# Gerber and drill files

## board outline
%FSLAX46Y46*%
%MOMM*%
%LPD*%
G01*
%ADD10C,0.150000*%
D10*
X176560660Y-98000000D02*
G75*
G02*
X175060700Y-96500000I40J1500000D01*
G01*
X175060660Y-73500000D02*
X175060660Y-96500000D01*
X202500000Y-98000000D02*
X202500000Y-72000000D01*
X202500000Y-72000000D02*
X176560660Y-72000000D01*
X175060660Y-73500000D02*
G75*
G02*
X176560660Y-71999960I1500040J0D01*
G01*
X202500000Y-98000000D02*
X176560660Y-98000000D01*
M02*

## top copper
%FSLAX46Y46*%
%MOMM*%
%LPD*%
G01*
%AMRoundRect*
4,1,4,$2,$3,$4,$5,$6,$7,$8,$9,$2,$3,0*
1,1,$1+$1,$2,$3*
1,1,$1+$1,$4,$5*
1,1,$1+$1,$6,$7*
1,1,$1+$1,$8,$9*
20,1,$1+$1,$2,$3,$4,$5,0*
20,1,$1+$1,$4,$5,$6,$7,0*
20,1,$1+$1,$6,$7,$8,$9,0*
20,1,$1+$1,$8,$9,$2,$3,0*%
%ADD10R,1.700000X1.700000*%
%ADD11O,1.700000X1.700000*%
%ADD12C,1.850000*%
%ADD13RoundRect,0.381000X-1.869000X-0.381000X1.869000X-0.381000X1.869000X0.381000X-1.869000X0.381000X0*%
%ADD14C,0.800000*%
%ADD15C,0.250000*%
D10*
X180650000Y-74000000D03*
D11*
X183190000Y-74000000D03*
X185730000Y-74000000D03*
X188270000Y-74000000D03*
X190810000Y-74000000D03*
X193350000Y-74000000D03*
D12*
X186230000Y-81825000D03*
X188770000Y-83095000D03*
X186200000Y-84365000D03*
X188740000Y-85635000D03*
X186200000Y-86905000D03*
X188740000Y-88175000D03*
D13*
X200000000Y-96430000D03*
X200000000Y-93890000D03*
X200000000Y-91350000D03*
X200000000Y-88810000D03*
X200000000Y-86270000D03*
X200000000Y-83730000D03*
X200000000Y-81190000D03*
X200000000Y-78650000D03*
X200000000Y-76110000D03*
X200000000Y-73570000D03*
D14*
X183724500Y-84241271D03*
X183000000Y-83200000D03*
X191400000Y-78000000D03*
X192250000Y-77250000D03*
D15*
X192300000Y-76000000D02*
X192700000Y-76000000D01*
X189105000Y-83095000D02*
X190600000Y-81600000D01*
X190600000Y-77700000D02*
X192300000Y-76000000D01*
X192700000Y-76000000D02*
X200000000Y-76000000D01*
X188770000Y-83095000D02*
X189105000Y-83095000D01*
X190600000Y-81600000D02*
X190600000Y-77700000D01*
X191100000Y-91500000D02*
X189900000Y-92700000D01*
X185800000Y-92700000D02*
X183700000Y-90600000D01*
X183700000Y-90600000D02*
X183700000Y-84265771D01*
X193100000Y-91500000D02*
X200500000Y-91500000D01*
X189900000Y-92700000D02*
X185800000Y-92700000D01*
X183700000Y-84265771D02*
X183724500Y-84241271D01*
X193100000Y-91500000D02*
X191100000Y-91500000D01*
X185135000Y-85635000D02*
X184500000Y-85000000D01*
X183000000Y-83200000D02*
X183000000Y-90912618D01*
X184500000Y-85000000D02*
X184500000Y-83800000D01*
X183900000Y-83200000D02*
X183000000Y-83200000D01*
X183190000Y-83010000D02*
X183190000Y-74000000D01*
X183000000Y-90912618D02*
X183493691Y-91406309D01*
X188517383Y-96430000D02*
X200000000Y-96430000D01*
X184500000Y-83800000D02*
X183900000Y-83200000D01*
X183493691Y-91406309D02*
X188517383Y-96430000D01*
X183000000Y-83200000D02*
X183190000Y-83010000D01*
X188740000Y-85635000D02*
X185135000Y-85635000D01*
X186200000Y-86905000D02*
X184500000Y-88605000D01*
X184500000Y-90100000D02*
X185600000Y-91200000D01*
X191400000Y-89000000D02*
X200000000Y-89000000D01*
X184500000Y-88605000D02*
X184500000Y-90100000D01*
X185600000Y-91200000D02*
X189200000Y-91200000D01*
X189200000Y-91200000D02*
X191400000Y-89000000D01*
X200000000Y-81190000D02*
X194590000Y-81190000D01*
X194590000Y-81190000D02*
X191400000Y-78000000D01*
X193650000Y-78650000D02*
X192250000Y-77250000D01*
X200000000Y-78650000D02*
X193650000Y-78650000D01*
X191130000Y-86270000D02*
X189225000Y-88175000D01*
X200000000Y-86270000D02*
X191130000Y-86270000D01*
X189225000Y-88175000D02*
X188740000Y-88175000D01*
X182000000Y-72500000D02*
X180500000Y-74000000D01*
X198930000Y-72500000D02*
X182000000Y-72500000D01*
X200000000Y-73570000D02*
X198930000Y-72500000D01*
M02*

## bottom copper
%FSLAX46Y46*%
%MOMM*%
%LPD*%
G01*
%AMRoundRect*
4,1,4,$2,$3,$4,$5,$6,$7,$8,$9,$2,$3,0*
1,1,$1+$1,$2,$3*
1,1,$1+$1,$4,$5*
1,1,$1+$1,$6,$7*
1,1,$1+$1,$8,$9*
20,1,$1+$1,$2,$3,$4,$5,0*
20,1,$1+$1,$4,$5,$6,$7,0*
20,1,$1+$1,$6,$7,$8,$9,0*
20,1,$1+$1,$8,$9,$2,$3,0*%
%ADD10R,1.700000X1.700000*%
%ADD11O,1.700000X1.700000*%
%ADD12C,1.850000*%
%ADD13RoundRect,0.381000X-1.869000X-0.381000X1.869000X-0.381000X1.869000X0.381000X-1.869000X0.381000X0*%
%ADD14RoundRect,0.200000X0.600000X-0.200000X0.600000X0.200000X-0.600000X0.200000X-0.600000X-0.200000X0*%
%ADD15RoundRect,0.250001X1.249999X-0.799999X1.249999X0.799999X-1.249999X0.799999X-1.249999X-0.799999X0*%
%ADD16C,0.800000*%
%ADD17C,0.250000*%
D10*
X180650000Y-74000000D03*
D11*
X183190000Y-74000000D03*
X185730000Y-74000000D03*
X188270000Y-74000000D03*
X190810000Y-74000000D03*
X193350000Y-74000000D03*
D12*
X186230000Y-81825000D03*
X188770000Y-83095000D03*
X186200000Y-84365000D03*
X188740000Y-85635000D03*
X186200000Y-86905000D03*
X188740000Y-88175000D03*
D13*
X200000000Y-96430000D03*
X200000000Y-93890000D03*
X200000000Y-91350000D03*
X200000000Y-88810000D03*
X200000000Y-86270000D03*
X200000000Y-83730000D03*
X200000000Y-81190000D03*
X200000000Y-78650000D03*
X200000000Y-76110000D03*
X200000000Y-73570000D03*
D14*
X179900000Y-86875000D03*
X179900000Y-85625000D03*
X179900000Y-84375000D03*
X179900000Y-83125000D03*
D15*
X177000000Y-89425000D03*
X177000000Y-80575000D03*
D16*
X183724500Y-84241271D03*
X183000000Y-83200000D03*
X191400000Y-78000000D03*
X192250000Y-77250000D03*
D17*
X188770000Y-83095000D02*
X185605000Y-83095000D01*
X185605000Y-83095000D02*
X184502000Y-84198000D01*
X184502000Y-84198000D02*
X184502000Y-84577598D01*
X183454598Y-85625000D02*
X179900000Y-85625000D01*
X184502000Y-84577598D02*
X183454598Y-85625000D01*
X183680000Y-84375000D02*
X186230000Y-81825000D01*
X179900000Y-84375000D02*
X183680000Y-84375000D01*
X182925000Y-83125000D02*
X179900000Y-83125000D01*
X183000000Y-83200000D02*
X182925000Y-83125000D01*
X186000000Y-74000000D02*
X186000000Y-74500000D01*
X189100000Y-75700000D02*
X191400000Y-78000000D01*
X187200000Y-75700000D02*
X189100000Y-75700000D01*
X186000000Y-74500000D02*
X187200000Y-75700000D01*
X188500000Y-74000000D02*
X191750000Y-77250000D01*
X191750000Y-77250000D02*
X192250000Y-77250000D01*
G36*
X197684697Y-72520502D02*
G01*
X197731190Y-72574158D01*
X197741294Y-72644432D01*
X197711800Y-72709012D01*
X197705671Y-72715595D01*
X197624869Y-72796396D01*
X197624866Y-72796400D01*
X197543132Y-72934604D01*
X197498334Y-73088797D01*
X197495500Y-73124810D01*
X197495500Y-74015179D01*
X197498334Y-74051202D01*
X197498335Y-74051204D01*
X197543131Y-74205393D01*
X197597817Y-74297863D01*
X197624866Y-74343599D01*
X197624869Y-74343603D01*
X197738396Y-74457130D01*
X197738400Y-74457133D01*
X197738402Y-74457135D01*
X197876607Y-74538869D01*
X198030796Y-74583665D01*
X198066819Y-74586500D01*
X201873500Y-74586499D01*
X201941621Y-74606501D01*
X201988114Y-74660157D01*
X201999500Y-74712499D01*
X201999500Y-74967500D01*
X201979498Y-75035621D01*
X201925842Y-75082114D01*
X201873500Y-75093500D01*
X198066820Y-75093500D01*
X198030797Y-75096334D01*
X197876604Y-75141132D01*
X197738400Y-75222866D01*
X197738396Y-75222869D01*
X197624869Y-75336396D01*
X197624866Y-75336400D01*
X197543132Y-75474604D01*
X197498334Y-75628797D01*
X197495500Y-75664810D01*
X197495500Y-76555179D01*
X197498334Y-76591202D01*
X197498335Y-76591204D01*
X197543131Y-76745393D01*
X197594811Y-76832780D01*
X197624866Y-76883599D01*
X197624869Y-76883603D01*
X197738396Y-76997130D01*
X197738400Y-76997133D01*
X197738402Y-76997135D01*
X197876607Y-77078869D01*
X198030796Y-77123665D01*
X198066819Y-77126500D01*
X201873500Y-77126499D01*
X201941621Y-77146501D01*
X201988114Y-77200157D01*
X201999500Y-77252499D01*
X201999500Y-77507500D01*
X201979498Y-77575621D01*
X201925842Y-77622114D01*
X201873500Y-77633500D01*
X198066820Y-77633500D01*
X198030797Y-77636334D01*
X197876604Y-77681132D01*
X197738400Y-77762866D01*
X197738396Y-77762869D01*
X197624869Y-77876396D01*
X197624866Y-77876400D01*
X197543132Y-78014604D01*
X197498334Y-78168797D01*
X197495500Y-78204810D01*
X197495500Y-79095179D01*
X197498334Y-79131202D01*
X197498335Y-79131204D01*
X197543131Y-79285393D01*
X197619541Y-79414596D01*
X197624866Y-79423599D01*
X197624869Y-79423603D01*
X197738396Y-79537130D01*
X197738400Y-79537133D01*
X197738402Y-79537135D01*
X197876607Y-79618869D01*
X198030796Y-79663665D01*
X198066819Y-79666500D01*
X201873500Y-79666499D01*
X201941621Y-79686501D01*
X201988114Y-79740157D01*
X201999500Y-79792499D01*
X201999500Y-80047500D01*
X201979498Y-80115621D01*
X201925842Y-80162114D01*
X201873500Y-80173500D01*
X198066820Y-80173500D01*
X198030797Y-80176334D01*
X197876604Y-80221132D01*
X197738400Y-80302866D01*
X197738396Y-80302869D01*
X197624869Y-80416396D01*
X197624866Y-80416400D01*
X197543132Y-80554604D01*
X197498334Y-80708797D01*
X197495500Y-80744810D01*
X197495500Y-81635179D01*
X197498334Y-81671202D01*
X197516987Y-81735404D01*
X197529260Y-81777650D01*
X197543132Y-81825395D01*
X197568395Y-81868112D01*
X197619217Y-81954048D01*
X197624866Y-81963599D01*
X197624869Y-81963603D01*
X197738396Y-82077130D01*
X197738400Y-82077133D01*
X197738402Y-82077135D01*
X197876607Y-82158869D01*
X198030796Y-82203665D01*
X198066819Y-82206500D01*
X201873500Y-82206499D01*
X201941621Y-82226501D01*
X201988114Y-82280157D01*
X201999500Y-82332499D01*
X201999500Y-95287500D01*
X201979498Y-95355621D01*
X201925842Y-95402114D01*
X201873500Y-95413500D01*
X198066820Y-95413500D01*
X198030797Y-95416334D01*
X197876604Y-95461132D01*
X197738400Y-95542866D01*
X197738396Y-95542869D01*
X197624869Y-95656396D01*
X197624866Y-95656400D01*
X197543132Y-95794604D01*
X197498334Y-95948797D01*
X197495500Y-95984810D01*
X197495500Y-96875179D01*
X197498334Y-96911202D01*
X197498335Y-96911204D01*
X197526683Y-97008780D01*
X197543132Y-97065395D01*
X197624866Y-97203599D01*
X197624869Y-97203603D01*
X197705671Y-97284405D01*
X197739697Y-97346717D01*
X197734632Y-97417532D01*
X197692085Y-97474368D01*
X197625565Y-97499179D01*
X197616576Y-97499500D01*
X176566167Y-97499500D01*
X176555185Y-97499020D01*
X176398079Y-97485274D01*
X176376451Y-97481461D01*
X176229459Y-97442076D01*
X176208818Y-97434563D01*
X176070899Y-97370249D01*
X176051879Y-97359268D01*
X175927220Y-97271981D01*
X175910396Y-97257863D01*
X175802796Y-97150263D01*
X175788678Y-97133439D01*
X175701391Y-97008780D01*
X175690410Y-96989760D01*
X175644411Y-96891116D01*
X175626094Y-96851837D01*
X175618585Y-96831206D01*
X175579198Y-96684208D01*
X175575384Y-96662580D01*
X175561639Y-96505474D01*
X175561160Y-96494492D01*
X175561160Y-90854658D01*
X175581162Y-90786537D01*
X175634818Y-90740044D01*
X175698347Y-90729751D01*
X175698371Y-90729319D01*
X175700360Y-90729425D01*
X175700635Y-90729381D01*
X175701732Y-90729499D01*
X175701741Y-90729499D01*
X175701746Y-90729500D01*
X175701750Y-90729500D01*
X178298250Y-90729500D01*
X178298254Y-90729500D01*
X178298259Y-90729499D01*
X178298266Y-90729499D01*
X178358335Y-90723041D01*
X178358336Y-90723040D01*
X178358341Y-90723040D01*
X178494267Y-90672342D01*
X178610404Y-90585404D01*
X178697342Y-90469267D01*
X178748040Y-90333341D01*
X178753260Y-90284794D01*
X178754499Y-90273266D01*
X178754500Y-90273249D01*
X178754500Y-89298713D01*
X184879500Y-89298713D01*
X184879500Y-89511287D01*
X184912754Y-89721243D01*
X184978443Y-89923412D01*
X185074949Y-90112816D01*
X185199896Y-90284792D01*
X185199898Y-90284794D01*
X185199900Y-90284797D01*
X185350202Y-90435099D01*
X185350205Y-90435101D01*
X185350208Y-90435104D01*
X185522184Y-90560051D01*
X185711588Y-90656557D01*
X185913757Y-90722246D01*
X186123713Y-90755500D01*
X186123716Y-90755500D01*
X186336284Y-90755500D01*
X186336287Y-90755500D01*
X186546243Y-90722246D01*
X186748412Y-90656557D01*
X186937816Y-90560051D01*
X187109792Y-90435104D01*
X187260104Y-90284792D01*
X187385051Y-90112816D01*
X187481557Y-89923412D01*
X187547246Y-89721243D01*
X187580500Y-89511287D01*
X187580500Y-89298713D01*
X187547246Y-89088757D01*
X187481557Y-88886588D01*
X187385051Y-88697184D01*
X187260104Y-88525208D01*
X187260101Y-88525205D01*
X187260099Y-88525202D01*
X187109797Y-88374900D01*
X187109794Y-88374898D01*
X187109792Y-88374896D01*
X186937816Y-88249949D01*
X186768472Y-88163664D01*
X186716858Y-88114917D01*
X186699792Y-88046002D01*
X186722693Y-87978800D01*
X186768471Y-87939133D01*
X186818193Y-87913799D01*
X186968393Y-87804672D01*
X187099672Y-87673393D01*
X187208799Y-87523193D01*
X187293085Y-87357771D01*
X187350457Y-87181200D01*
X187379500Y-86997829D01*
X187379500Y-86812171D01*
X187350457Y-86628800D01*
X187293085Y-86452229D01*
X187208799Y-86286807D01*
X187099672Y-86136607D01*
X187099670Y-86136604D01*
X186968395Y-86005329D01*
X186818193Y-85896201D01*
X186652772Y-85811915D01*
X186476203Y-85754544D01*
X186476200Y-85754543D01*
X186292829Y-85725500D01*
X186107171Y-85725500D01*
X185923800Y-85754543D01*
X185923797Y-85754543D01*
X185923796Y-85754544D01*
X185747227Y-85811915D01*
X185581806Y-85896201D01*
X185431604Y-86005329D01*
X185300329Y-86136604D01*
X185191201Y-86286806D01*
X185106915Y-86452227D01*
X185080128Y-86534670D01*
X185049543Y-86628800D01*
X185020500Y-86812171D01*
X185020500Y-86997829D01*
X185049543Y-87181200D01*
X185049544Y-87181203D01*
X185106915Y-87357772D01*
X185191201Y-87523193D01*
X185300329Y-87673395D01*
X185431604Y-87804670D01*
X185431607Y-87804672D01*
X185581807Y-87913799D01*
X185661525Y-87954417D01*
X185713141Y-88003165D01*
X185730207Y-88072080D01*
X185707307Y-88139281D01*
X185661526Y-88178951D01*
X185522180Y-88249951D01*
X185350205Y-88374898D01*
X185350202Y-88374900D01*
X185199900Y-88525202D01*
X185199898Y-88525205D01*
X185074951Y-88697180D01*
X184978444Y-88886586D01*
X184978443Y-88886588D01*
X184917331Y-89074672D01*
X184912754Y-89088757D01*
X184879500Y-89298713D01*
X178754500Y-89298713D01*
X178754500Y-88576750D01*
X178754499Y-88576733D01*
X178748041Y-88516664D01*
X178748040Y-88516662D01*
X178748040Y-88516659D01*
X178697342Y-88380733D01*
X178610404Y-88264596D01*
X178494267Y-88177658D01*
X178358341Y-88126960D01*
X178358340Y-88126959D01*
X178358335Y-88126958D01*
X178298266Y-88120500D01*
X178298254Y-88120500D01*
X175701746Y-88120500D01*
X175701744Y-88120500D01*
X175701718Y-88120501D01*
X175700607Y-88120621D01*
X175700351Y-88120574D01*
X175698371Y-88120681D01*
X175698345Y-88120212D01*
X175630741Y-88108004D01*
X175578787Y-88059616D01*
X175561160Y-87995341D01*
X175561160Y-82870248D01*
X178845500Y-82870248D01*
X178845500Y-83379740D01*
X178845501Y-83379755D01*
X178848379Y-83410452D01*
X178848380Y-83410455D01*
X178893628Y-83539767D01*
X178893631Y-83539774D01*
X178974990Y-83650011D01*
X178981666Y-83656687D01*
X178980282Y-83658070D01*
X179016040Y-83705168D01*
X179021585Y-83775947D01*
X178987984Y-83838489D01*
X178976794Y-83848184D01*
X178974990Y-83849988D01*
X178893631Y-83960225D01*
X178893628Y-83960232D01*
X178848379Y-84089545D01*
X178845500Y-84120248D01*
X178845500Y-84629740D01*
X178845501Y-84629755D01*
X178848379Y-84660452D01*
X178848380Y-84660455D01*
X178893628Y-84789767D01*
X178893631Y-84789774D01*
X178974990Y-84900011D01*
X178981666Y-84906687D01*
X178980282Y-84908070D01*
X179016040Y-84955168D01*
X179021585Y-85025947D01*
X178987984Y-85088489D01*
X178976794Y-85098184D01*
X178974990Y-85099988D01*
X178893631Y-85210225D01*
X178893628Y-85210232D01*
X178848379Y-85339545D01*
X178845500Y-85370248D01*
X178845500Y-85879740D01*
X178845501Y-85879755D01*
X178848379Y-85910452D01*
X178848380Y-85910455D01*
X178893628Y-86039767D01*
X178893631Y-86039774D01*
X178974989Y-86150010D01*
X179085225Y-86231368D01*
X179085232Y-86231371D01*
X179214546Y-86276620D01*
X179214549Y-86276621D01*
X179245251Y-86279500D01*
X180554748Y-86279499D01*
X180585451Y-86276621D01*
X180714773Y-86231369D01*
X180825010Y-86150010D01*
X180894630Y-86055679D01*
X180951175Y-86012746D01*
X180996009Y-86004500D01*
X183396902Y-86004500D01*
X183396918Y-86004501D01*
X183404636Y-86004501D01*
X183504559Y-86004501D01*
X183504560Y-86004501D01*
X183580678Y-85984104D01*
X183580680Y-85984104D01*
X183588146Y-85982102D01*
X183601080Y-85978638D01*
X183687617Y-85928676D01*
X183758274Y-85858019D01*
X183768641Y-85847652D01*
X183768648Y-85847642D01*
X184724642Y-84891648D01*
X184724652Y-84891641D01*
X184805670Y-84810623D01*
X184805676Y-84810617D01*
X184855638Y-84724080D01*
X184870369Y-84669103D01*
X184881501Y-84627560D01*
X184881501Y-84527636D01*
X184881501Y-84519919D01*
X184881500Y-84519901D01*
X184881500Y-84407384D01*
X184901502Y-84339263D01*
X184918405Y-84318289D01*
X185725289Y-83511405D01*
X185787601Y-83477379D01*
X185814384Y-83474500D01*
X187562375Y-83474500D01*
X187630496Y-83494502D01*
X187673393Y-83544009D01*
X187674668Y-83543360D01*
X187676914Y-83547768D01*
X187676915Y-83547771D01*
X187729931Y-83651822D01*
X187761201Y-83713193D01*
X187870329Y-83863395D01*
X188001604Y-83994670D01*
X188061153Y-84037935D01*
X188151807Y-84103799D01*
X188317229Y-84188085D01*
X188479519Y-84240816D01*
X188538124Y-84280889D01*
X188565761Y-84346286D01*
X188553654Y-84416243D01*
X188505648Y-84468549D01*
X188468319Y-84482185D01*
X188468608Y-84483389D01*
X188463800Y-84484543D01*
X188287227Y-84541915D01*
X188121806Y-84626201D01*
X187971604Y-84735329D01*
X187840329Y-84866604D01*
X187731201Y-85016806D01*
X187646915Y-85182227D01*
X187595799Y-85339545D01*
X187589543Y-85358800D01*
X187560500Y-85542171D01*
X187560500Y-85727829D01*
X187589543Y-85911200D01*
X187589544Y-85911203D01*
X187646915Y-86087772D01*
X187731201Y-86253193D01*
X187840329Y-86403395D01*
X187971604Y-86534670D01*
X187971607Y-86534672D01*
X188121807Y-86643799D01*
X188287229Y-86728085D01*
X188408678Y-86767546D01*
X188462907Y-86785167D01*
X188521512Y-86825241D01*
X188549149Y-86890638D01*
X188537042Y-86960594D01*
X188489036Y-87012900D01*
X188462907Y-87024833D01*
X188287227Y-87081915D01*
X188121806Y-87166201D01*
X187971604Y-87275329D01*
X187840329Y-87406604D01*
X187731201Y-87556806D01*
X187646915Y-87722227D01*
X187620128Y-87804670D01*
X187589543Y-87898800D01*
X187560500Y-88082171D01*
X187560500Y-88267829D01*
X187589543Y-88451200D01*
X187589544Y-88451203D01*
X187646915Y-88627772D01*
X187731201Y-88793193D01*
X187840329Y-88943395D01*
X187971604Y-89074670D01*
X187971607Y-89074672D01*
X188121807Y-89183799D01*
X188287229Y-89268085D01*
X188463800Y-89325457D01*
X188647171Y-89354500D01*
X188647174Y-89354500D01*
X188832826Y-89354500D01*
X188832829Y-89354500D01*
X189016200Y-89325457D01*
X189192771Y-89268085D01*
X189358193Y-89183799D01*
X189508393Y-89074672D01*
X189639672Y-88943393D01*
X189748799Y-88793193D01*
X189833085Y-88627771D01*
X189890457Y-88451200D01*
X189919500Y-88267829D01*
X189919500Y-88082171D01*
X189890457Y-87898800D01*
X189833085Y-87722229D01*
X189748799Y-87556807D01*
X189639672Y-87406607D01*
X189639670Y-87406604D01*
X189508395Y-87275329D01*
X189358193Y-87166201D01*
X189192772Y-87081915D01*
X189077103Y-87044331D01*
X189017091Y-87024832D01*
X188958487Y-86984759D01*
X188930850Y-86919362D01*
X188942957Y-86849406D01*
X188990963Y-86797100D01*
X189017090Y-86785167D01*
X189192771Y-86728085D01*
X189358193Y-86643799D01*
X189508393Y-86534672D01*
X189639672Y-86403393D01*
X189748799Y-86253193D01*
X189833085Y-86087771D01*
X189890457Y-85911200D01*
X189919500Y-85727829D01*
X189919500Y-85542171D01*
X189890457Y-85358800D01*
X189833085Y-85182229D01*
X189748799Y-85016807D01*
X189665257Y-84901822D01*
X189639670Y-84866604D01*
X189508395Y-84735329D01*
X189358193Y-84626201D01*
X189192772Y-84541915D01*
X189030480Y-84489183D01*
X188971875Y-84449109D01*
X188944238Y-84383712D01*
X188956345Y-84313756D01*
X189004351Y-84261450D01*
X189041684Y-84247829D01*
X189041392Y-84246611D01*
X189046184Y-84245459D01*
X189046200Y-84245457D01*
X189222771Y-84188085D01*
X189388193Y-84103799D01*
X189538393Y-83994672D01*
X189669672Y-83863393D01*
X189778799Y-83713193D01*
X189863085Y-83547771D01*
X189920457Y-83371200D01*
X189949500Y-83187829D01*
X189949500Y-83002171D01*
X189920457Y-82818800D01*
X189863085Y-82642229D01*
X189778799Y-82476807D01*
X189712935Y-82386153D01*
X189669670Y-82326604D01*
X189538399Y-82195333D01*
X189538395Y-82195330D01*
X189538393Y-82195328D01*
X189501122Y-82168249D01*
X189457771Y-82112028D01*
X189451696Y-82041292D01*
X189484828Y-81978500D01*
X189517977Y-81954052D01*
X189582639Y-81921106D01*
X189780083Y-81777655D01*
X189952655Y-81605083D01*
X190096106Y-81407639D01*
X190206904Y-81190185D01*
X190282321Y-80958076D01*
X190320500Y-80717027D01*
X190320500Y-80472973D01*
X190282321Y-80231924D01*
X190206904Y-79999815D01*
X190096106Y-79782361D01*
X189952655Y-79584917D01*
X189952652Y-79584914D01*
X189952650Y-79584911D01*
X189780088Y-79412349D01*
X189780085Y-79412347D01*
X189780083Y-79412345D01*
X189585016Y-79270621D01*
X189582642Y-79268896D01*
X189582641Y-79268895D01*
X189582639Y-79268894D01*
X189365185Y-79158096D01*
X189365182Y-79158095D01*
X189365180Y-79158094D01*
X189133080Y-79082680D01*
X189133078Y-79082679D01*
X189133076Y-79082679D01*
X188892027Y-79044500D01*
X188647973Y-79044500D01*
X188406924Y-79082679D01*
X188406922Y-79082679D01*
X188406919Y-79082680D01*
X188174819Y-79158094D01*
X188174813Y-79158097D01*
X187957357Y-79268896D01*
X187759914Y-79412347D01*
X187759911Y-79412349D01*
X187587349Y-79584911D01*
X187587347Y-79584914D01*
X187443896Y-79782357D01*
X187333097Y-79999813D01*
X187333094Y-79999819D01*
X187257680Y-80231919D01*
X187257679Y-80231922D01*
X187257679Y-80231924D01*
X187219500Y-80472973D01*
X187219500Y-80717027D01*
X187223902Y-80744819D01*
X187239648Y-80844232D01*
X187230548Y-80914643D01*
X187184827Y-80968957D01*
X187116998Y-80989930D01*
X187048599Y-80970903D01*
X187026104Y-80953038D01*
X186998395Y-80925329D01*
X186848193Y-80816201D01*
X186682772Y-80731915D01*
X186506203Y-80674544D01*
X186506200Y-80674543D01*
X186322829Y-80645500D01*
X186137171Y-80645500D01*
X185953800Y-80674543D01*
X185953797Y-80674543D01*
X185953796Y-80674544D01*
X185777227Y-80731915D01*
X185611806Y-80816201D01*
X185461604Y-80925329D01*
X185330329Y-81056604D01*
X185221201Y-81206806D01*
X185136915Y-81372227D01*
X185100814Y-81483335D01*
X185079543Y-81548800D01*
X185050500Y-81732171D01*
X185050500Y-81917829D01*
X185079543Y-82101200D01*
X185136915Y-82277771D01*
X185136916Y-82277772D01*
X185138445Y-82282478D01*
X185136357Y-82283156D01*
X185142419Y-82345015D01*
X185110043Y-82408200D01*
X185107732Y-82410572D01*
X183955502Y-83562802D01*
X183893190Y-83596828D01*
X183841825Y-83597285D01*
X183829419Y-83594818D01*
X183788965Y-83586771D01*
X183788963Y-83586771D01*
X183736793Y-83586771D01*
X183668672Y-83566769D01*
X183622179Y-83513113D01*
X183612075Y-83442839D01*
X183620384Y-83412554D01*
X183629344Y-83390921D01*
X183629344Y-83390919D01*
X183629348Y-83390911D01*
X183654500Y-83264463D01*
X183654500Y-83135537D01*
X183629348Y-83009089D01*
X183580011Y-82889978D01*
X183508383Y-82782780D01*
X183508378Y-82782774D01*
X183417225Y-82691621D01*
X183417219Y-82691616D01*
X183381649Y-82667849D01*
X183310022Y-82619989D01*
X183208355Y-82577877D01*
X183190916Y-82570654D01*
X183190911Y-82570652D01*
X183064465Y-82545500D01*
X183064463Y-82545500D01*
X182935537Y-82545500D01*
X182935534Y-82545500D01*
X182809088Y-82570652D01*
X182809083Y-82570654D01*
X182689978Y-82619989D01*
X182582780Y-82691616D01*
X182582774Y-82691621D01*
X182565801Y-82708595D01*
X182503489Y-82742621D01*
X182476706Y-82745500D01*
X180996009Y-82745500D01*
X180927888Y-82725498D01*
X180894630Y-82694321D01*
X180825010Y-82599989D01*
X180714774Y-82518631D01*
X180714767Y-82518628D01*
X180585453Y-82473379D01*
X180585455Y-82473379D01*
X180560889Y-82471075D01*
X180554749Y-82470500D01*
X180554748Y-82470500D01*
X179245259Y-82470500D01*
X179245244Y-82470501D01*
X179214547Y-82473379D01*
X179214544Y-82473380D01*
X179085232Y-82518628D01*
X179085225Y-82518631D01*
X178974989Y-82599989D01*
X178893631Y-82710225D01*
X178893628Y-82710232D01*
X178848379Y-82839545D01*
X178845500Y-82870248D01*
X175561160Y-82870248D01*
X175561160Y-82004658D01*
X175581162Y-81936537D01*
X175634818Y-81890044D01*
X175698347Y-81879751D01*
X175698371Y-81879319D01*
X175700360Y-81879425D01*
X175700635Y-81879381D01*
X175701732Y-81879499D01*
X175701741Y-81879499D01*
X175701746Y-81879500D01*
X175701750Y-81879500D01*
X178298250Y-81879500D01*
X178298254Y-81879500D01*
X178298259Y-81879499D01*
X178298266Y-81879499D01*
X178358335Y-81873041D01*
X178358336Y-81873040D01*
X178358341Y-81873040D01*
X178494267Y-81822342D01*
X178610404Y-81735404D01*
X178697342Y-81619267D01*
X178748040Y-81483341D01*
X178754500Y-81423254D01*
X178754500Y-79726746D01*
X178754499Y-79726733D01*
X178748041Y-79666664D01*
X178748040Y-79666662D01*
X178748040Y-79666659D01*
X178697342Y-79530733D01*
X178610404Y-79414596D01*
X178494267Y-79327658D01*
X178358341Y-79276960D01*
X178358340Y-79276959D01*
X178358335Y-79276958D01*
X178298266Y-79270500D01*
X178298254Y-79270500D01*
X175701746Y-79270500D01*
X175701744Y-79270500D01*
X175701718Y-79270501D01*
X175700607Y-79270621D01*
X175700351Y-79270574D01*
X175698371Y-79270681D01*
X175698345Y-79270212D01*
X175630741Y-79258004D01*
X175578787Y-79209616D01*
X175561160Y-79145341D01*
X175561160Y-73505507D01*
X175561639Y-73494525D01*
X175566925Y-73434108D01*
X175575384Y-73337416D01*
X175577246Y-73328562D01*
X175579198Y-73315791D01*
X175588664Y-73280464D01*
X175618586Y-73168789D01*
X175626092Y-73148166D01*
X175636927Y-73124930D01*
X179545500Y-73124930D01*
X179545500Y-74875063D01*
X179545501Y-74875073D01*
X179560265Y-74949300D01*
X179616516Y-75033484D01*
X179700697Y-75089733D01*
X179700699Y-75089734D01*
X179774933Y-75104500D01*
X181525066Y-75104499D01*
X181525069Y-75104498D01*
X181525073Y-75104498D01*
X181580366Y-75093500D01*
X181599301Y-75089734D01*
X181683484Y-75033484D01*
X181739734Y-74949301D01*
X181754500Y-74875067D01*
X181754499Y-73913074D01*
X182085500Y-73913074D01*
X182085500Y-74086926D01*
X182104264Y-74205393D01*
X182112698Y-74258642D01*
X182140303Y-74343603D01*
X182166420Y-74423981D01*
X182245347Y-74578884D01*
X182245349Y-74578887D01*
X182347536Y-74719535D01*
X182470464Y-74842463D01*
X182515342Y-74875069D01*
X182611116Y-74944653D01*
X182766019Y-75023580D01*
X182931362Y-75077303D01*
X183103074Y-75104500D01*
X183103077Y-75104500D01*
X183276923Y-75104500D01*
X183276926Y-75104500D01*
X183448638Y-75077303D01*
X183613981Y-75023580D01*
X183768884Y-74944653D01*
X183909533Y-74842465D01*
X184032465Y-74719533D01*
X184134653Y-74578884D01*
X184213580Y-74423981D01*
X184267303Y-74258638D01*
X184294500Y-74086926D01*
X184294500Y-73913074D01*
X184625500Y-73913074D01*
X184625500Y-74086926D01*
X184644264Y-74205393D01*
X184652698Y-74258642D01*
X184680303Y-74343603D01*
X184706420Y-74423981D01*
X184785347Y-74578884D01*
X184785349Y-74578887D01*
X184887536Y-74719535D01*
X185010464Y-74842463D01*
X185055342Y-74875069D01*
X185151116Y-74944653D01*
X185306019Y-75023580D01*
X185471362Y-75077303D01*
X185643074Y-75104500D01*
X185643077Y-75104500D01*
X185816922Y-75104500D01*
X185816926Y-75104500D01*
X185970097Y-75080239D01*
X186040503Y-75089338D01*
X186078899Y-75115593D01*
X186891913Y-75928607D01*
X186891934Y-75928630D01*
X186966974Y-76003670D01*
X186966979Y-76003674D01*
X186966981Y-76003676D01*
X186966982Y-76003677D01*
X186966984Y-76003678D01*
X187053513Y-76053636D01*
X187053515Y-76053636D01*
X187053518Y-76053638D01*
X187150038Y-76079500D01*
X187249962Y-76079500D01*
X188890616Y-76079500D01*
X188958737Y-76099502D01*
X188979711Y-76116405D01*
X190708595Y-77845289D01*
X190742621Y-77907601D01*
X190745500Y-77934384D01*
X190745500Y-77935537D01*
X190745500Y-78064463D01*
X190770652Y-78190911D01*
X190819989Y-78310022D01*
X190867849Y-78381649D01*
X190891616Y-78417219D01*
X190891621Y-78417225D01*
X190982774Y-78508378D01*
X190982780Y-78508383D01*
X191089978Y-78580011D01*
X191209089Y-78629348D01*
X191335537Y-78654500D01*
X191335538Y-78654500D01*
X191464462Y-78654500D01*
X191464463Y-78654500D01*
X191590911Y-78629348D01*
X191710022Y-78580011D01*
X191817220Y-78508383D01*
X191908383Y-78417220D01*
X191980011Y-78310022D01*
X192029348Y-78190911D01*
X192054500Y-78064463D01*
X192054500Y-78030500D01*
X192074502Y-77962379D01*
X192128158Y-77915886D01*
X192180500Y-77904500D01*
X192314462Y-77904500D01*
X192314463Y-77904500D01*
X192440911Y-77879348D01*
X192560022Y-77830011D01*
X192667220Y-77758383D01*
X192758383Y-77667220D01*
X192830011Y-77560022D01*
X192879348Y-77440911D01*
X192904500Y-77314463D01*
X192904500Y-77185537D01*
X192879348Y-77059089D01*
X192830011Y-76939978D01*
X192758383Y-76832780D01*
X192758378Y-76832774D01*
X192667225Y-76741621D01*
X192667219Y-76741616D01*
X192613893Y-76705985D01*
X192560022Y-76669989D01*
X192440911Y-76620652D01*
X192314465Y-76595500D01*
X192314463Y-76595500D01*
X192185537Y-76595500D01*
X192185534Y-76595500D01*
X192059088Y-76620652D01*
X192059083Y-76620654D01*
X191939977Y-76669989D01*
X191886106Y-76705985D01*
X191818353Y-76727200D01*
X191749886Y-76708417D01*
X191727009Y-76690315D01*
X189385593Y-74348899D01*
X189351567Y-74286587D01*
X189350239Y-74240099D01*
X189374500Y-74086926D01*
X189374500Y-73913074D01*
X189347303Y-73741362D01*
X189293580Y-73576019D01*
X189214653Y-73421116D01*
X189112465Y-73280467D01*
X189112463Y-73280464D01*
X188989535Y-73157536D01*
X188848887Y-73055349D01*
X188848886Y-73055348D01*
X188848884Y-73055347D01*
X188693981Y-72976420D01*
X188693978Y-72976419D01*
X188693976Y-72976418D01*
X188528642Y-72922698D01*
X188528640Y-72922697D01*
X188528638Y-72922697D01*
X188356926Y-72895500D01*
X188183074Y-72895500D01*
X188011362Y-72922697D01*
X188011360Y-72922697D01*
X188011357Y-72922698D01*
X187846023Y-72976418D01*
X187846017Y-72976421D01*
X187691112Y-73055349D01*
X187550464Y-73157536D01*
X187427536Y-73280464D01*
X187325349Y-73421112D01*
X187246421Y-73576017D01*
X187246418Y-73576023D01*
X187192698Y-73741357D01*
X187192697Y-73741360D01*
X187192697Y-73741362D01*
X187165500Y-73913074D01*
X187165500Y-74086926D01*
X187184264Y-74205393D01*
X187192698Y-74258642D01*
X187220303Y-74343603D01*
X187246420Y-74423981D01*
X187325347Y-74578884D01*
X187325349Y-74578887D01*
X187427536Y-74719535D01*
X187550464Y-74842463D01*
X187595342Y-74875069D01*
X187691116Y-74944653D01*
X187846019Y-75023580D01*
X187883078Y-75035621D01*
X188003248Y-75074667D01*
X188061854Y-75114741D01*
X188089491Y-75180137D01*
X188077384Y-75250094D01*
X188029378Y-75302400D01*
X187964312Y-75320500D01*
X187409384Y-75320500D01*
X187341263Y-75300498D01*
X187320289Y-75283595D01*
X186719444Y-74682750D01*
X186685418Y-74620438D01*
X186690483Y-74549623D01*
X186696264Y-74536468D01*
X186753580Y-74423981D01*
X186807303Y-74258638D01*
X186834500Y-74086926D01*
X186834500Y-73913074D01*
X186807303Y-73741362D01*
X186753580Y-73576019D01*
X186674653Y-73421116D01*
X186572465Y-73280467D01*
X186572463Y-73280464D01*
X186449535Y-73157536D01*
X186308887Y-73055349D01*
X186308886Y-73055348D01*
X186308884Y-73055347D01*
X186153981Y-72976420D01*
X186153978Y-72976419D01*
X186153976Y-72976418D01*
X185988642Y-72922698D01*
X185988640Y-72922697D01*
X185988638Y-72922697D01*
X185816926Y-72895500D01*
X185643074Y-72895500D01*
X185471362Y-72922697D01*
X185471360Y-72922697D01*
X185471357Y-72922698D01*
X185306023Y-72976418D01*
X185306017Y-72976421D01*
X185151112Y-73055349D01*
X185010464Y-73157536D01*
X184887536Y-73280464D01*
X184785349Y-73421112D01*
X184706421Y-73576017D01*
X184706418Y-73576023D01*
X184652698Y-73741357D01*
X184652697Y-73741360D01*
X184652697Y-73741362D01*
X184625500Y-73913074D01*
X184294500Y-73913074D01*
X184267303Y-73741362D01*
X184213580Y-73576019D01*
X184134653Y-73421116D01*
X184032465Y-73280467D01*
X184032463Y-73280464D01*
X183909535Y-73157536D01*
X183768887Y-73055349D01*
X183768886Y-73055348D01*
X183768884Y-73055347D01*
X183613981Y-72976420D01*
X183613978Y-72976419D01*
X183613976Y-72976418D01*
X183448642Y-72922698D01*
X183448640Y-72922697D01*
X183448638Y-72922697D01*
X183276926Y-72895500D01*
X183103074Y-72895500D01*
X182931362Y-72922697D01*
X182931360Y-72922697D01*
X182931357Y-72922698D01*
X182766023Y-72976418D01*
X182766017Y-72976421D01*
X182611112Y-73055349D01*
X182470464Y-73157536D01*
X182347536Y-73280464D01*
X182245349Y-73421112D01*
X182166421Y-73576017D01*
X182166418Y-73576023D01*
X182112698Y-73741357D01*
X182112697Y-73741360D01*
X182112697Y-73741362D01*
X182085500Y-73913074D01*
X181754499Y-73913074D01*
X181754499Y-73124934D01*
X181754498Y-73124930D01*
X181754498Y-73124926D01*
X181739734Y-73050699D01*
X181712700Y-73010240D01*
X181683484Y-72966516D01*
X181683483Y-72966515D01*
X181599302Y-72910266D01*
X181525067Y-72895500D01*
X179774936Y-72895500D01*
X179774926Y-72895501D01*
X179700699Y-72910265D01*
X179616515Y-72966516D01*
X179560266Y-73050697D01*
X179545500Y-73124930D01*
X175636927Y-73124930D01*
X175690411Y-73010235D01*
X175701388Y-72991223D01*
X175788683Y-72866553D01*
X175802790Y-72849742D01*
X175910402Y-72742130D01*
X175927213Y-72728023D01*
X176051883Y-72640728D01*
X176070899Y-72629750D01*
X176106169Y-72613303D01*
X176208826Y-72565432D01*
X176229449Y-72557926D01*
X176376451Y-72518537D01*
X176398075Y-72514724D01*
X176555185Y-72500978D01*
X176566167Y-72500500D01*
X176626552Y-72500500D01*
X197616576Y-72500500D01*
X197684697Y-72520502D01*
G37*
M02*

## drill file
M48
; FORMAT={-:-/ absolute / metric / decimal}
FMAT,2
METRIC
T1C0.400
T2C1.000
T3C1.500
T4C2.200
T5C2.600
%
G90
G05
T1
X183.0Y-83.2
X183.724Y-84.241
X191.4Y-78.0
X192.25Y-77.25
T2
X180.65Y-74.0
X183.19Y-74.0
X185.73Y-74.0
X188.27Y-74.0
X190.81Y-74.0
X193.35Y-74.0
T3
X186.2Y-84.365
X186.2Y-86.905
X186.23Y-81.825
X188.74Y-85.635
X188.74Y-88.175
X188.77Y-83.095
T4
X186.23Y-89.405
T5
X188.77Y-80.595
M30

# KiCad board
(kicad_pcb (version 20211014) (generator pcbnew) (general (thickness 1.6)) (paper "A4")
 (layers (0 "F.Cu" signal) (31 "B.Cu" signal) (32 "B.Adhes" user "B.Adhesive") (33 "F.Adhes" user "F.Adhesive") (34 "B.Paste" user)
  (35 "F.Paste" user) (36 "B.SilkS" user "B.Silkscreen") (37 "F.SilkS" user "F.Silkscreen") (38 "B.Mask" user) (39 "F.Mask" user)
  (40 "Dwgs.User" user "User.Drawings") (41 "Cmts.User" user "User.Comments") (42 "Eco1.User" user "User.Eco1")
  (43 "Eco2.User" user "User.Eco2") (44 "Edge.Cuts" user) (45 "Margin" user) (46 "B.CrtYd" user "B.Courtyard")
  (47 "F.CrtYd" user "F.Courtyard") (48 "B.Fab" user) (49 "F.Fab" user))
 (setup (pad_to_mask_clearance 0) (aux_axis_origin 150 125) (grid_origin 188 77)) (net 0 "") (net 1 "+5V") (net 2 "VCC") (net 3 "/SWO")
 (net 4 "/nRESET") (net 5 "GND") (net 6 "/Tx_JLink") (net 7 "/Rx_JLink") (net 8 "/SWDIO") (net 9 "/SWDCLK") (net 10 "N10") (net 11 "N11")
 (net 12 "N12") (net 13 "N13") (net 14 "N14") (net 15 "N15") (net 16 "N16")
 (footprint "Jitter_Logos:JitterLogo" (layer "F.Cu") (at 179.25 90)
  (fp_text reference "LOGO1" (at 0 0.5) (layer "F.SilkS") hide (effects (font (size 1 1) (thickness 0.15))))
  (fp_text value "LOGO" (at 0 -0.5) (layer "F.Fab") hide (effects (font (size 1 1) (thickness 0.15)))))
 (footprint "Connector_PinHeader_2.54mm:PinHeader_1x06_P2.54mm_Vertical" (layer "F.Cu") (at 180.65 74 90)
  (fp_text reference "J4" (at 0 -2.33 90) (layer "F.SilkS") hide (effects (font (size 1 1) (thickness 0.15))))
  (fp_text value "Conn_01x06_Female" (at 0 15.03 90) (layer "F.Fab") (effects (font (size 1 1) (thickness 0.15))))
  (pad "1" thru_hole rect (at 0 0 90) (size 1.7 1.7) (drill 1) (layers *.Cu *.Mask) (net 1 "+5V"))
  (pad "2" thru_hole oval (at 0 2.54 90) (size 1.7 1.7) (drill 1) (layers *.Cu *.Mask) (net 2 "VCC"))
  (pad "3" thru_hole oval (at 0 5.08 90) (size 1.7 1.7) (drill 1) (layers *.Cu *.Mask) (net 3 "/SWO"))
  (pad "4" thru_hole oval (at 0 7.62 90) (size 1.7 1.7) (drill 1) (layers *.Cu *.Mask) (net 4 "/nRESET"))
  (pad "5" thru_hole oval (at 0 10.16 90) (size 1.7 1.7) (drill 1) (layers *.Cu *.Mask) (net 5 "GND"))
  (pad "6" thru_hole oval (at 0 12.7 90) (size 1.7 1.7) (drill 1) (layers *.Cu *.Mask) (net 5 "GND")))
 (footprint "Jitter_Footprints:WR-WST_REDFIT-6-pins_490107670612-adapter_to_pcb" (layer "F.Cu") (at 187.5 85 90)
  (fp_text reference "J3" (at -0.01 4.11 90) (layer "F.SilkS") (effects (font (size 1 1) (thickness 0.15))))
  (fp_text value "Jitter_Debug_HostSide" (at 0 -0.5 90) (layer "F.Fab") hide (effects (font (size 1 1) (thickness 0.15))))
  (pad "" np_thru_hole circle locked (at 4.405 1.27 90) (size 2.6 2.6) (drill 2.6) (layers *.Cu *.Mask))
  (pad "" np_thru_hole circle locked (at -4.405 -1.27 90) (size 2.2 2.2) (drill 2.2) (layers *.Cu *.Mask))
  (pad "1" thru_hole circle locked (at 3.175 -1.27 90) (size 1.85 1.85) (drill 1.5) (layers *.Cu *.Mask) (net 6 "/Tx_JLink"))
  (pad "2" thru_hole circle locked (at 1.905 1.27 90) (size 1.85 1.85) (drill 1.5) (layers *.Cu *.Mask) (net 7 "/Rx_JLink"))
  (pad "3" thru_hole circle locked (at 0.635 -1.3 90) (size 1.85 1.85) (drill 1.5) (layers *.Cu *.Mask) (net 5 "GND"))
  (pad "4" thru_hole circle locked (at -0.635 1.24 90) (size 1.85 1.85) (drill 1.5) (layers *.Cu *.Mask) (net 2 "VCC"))
  (pad "5" thru_hole circle locked (at -1.905 -1.3 90) (size 1.85 1.85) (drill 1.5) (layers *.Cu *.Mask) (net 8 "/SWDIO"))
  (pad "6" thru_hole circle locked (at -3.175 1.24 90) (size 1.85 1.85) (drill 1.5) (layers *.Cu *.Mask) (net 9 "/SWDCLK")))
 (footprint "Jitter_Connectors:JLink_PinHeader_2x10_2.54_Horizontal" (layer "F.Cu") (at 200 85)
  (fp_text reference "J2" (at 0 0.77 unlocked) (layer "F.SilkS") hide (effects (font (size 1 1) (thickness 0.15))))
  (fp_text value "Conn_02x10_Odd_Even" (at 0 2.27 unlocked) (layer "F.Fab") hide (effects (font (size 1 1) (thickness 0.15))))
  (pad "1" smd roundrect (at 0 11.43) (size 4.5 1.524) (layers "F.Cu" "F.Paste" "F.Mask") (roundrect_rratio 0.25) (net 2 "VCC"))
  (pad "2" smd roundrect (at 0 11.43) (size 4.5 1.524) (layers "B.Cu" "B.Paste" "B.Mask") (roundrect_rratio 0.25) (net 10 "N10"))
  (pad "3" smd roundrect (at 0 8.89) (size 4.5 1.524) (layers "F.Cu" "F.Paste" "F.Mask") (roundrect_rratio 0.25) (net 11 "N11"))
  (pad "4" smd roundrect (at 0 8.89) (size 4.5 1.524) (layers "B.Cu" "B.Paste" "B.Mask") (roundrect_rratio 0.25) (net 5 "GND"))
  (pad "5" smd roundrect (at 0 6.35) (size 4.5 1.524) (layers "F.Cu" "F.Paste" "F.Mask") (roundrect_rratio 0.25) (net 6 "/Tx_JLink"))
  (pad "6" smd roundrect (at 0 6.35) (size 4.5 1.524) (layers "B.Cu" "B.Paste" "B.Mask") (roundrect_rratio 0.25) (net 5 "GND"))
  (pad "7" smd roundrect (at 0 3.81) (size 4.5 1.524) (layers "F.Cu" "F.Paste" "F.Mask") (roundrect_rratio 0.25) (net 8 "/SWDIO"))
  (pad "8" smd roundrect (at 0 3.81) (size 4.5 1.524) (layers "B.Cu" "B.Paste" "B.Mask") (roundrect_rratio 0.25) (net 5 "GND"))
  (pad "9" smd roundrect (at 0 1.27) (size 4.5 1.524) (layers "F.Cu" "F.Paste" "F.Mask") (roundrect_rratio 0.25) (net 9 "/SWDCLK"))
  (pad "10" smd roundrect (at 0 1.27) (size 4.5 1.524) (layers "B.Cu" "B.Paste" "B.Mask") (roundrect_rratio 0.25) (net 5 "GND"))
  (pad "11" smd roundrect (at 0 -1.27) (size 4.5 1.524) (layers "F.Cu" "F.Paste" "F.Mask") (roundrect_rratio 0.25) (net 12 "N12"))
  (pad "12" smd roundrect (at 0 -1.27) (size 4.5 1.524) (layers "B.Cu" "B.Paste" "B.Mask") (roundrect_rratio 0.25) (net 5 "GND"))
  (pad "13" smd roundrect (at 0 -3.81) (size 4.5 1.524) (layers "F.Cu" "F.Paste" "F.Mask") (roundrect_rratio 0.25) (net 3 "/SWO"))
  (pad "14" smd roundrect (at 0 -3.81) (size 4.5 1.524) (layers "B.Cu" "B.Paste" "B.Mask") (roundrect_rratio 0.25) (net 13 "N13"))
  (pad "15" smd roundrect (at 0 -6.35) (size 4.5 1.524) (layers "F.Cu" "F.Paste" "F.Mask") (roundrect_rratio 0.25) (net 4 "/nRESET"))
  (pad "16" smd roundrect (at 0 -6.35) (size 4.5 1.524) (layers "B.Cu" "B.Paste" "B.Mask") (roundrect_rratio 0.25) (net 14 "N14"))
  (pad "17" smd roundrect (at 0 -8.89) (size 4.5 1.524) (layers "F.Cu" "F.Paste" "F.Mask") (roundrect_rratio 0.25) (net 7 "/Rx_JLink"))
  (pad "18" smd roundrect (at 0 -8.89) (size 4.5 1.524) (layers "B.Cu" "B.Paste" "B.Mask") (roundrect_rratio 0.25) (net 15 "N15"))
  (pad "19" smd roundrect (at 0 -11.43) (size 4.5 1.524) (layers "F.Cu" "F.Paste" "F.Mask") (roundrect_rratio 0.25) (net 1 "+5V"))
  (pad "20" smd roundrect (at 0 -11.43) (size 4.5 1.524) (layers "B.Cu" "B.Paste" "B.Mask") (roundrect_rratio 0.25) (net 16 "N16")))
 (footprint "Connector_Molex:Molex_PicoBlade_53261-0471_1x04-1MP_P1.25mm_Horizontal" (layer "B.Cu") (at 177.5 85 90)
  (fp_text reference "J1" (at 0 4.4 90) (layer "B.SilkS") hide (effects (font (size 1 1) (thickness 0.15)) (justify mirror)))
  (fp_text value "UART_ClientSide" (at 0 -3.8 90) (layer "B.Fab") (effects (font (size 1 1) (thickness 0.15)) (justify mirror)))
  (pad "1" smd roundrect (at -1.875 2.4 90) (size 0.8 1.6) (layers "B.Cu" "B.Paste" "B.Mask") (roundrect_rratio 0.25) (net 5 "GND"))
  (pad "2" smd roundrect (at -0.625 2.4 90) (size 0.8 1.6) (layers "B.Cu" "B.Paste" "B.Mask") (roundrect_rratio 0.25) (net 7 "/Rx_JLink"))
  (pad "3" smd roundrect (at 0.625 2.4 90) (size 0.8 1.6) (layers "B.Cu" "B.Paste" "B.Mask") (roundrect_rratio 0.25) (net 6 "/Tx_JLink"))
  (pad "4" smd roundrect (at 1.875 2.4 90) (size 0.8 1.6) (layers "B.Cu" "B.Paste" "B.Mask") (roundrect_rratio 0.25) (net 2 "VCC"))
  (pad "MP" smd roundrect (at -4.425 -0.5 90) (size 2.1 3) (layers "B.Cu" "B.Paste" "B.Mask") (roundrect_rratio 0.1190480952))
  (pad "MP" smd roundrect (at 4.425 -0.5 90) (size 2.1 3) (layers "B.Cu" "B.Paste" "B.Mask") (roundrect_rratio 0.1190480952)))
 (gr_arc (start 176.56066 98) (mid 175.5 97.56066) (end 175.06066 96.5) (layer "Edge.Cuts") (width 0.15))
 (gr_line (start 175.06066 73.5) (end 175.06066 96.5) (layer "Edge.Cuts") (width 0.15))
 (gr_line (start 202.5 98) (end 202.5 72) (layer "Edge.Cuts") (width 0.15))
 (gr_line (start 202.5 72) (end 176.56066 72) (layer "Edge.Cuts") (width 0.15))
 (gr_arc (start 175.06066 73.5) (mid 175.5 72.43934) (end 176.56066 72) (layer "Edge.Cuts") (width 0.15))
 (gr_line (start 202.5 98) (end 176.56066 98) (layer "Edge.Cuts") (width 0.15))
 (segment (start 192.3 76) (end 192.7 76) (width 0.25) (layer "F.Cu") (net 7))
 (segment (start 189.105 83.095) (end 190.6 81.6) (width 0.25) (layer "F.Cu") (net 7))
 (segment (start 190.6 77.7) (end 192.3 76) (width 0.25) (layer "F.Cu") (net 7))
 (segment (start 192.7 76) (end 200 76) (width 0.25) (layer "F.Cu") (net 7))
 (segment (start 188.77 83.095) (end 189.105 83.095) (width 0.25) (layer "F.Cu") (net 7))
 (segment (start 190.6 81.6) (end 190.6 77.7) (width 0.25) (layer "F.Cu") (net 7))
 (segment (start 188.77 83.095) (end 185.605 83.095) (width 0.25) (layer "B.Cu") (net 7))
 (segment (start 185.605 83.095) (end 184.502 84.198) (width 0.25) (layer "B.Cu") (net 7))
 (segment (start 184.502 84.198) (end 184.502 84.577598) (width 0.25) (layer "B.Cu") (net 7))
 (segment (start 183.454598 85.625) (end 179.9 85.625) (width 0.25) (layer "B.Cu") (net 7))
 (segment (start 184.502 84.577598) (end 183.454598 85.625) (width 0.25) (layer "B.Cu") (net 7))
 (segment (start 191.1 91.5) (end 189.9 92.7) (width 0.25) (layer "F.Cu") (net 6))
 (segment (start 185.8 92.7) (end 183.7 90.6) (width 0.25) (layer "F.Cu") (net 6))
 (segment (start 183.7 90.6) (end 183.7 84.265771) (width 0.25) (layer "F.Cu") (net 6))
 (segment (start 193.1 91.5) (end 200.5 91.5) (width 0.25) (layer "F.Cu") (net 6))
 (segment (start 189.9 92.7) (end 185.8 92.7) (width 0.25) (layer "F.Cu") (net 6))
 (segment (start 183.7 84.265771) (end 183.7245 84.241271) (width 0.25) (layer "F.Cu") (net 6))
 (segment (start 193.1 91.5) (end 191.1 91.5) (width 0.25) (layer "F.Cu") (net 6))
 (via (at 183.7245 84.241271) (size 0.8) (drill 0.4) (layers "F.Cu" "B.Cu") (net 6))
 (segment (start 183.68 84.375) (end 186.23 81.825) (width 0.25) (layer "B.Cu") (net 6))
 (segment (start 179.9 84.375) (end 183.68 84.375) (width 0.25) (layer "B.Cu") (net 6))
 (segment (start 185.135 85.635) (end 184.5 85) (width 0.25) (layer "F.Cu") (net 2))
 (segment (start 183 83.2) (end 183 90.912618) (width 0.25) (layer "F.Cu") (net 2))
 (segment (start 184.5 85) (end 184.5 83.8) (width 0.25) (layer "F.Cu") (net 2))
 (segment (start 183.9 83.2) (end 183 83.2) (width 0.25) (layer "F.Cu") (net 2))
 (segment (start 183.19 83.01) (end 183.19 74) (width 0.25) (layer "F.Cu") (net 2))
 (segment (start 183 90.912618) (end 183.493691 91.406309) (width 0.25) (layer "F.Cu") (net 2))
 (segment (start 188.517383 96.43) (end 200 96.43) (width 0.25) (layer "F.Cu") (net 2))
 (segment (start 184.5 83.8) (end 183.9 83.2) (width 0.25) (layer "F.Cu") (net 2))
 (segment (start 183.493691 91.406309) (end 188.517383 96.43) (width 0.25) (layer "F.Cu") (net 2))
 (segment (start 183 83.2) (end 183.19 83.01) (width 0.25) (layer "F.Cu") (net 2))
 (segment (start 188.74 85.635) (end 185.135 85.635) (width 0.25) (layer "F.Cu") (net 2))
 (via (at 183 83.2) (size 0.8) (drill 0.4) (layers "F.Cu" "B.Cu") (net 2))
 (segment (start 182.925 83.125) (end 179.9 83.125) (width 0.25) (layer "B.Cu") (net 2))
 (segment (start 183 83.2) (end 182.925 83.125) (width 0.25) (layer "B.Cu") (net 2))
 (segment (start 186.2 86.905) (end 184.5 88.605) (width 0.25) (layer "F.Cu") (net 8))
 (segment (start 184.5 90.1) (end 185.6 91.2) (width 0.25) (layer "F.Cu") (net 8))
 (segment (start 191.4 89) (end 200 89) (width 0.25) (layer "F.Cu") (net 8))
 (segment (start 184.5 88.605) (end 184.5 90.1) (width 0.25) (layer "F.Cu") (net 8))
 (segment (start 185.6 91.2) (end 189.2 91.2) (width 0.25) (layer "F.Cu") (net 8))
 (segment (start 189.2 91.2) (end 191.4 89) (width 0.25) (layer "F.Cu") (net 8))
 (segment (start 200 81.19) (end 194.59 81.19) (width 0.25) (layer "F.Cu") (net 3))
 (segment (start 194.59 81.19) (end 191.4 78) (width 0.25) (layer "F.Cu") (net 3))
 (via (at 191.4 78) (size 0.8) (drill 0.4) (layers "F.Cu" "B.Cu") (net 3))
 (segment (start 186 74) (end 186 74.5) (width 0.25) (layer "B.Cu") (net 3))
 (segment (start 189.1 75.7) (end 191.4 78) (width 0.25) (layer "B.Cu") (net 3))
 (segment (start 187.2 75.7) (end 189.1 75.7) (width 0.25) (layer "B.Cu") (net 3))
 (segment (start 186 74.5) (end 187.2 75.7) (width 0.25) (layer "B.Cu") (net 3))
 (segment (start 193.65 78.65) (end 192.25 77.25) (width 0.25) (layer "F.Cu") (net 4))
 (segment (start 200 78.65) (end 193.65 78.65) (width 0.25) (layer "F.Cu") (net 4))
 (via (at 192.25 77.25) (size 0.8) (drill 0.4) (layers "F.Cu" "B.Cu") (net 4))
 (segment (start 188.5 74) (end 191.75 77.25) (width 0.25) (layer "B.Cu") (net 4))
 (segment (start 191.75 77.25) (end 192.25 77.25) (width 0.25) (layer "B.Cu") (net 4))
 (segment (start 191.13 86.27) (end 189.225 88.175) (width 0.25) (layer "F.Cu") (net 9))
 (segment (start 200 86.27) (end 191.13 86.27) (width 0.25) (layer "F.Cu") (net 9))
 (segment (start 189.225 88.175) (end 188.74 88.175) (width 0.25) (layer "F.Cu") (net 9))
 (segment (start 182 72.5) (end 180.5 74) (width 0.25) (layer "F.Cu") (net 1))
 (segment (start 198.93 72.5) (end 182 72.5) (width 0.25) (layer "F.Cu") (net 1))
 (segment (start 200 73.57) (end 198.93 72.5) (width 0.25) (layer "F.Cu") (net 1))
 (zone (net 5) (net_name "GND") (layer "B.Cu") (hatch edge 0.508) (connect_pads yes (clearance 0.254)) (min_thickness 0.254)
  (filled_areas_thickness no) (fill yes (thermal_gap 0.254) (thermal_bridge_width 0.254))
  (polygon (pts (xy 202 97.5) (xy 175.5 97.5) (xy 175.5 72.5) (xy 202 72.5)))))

